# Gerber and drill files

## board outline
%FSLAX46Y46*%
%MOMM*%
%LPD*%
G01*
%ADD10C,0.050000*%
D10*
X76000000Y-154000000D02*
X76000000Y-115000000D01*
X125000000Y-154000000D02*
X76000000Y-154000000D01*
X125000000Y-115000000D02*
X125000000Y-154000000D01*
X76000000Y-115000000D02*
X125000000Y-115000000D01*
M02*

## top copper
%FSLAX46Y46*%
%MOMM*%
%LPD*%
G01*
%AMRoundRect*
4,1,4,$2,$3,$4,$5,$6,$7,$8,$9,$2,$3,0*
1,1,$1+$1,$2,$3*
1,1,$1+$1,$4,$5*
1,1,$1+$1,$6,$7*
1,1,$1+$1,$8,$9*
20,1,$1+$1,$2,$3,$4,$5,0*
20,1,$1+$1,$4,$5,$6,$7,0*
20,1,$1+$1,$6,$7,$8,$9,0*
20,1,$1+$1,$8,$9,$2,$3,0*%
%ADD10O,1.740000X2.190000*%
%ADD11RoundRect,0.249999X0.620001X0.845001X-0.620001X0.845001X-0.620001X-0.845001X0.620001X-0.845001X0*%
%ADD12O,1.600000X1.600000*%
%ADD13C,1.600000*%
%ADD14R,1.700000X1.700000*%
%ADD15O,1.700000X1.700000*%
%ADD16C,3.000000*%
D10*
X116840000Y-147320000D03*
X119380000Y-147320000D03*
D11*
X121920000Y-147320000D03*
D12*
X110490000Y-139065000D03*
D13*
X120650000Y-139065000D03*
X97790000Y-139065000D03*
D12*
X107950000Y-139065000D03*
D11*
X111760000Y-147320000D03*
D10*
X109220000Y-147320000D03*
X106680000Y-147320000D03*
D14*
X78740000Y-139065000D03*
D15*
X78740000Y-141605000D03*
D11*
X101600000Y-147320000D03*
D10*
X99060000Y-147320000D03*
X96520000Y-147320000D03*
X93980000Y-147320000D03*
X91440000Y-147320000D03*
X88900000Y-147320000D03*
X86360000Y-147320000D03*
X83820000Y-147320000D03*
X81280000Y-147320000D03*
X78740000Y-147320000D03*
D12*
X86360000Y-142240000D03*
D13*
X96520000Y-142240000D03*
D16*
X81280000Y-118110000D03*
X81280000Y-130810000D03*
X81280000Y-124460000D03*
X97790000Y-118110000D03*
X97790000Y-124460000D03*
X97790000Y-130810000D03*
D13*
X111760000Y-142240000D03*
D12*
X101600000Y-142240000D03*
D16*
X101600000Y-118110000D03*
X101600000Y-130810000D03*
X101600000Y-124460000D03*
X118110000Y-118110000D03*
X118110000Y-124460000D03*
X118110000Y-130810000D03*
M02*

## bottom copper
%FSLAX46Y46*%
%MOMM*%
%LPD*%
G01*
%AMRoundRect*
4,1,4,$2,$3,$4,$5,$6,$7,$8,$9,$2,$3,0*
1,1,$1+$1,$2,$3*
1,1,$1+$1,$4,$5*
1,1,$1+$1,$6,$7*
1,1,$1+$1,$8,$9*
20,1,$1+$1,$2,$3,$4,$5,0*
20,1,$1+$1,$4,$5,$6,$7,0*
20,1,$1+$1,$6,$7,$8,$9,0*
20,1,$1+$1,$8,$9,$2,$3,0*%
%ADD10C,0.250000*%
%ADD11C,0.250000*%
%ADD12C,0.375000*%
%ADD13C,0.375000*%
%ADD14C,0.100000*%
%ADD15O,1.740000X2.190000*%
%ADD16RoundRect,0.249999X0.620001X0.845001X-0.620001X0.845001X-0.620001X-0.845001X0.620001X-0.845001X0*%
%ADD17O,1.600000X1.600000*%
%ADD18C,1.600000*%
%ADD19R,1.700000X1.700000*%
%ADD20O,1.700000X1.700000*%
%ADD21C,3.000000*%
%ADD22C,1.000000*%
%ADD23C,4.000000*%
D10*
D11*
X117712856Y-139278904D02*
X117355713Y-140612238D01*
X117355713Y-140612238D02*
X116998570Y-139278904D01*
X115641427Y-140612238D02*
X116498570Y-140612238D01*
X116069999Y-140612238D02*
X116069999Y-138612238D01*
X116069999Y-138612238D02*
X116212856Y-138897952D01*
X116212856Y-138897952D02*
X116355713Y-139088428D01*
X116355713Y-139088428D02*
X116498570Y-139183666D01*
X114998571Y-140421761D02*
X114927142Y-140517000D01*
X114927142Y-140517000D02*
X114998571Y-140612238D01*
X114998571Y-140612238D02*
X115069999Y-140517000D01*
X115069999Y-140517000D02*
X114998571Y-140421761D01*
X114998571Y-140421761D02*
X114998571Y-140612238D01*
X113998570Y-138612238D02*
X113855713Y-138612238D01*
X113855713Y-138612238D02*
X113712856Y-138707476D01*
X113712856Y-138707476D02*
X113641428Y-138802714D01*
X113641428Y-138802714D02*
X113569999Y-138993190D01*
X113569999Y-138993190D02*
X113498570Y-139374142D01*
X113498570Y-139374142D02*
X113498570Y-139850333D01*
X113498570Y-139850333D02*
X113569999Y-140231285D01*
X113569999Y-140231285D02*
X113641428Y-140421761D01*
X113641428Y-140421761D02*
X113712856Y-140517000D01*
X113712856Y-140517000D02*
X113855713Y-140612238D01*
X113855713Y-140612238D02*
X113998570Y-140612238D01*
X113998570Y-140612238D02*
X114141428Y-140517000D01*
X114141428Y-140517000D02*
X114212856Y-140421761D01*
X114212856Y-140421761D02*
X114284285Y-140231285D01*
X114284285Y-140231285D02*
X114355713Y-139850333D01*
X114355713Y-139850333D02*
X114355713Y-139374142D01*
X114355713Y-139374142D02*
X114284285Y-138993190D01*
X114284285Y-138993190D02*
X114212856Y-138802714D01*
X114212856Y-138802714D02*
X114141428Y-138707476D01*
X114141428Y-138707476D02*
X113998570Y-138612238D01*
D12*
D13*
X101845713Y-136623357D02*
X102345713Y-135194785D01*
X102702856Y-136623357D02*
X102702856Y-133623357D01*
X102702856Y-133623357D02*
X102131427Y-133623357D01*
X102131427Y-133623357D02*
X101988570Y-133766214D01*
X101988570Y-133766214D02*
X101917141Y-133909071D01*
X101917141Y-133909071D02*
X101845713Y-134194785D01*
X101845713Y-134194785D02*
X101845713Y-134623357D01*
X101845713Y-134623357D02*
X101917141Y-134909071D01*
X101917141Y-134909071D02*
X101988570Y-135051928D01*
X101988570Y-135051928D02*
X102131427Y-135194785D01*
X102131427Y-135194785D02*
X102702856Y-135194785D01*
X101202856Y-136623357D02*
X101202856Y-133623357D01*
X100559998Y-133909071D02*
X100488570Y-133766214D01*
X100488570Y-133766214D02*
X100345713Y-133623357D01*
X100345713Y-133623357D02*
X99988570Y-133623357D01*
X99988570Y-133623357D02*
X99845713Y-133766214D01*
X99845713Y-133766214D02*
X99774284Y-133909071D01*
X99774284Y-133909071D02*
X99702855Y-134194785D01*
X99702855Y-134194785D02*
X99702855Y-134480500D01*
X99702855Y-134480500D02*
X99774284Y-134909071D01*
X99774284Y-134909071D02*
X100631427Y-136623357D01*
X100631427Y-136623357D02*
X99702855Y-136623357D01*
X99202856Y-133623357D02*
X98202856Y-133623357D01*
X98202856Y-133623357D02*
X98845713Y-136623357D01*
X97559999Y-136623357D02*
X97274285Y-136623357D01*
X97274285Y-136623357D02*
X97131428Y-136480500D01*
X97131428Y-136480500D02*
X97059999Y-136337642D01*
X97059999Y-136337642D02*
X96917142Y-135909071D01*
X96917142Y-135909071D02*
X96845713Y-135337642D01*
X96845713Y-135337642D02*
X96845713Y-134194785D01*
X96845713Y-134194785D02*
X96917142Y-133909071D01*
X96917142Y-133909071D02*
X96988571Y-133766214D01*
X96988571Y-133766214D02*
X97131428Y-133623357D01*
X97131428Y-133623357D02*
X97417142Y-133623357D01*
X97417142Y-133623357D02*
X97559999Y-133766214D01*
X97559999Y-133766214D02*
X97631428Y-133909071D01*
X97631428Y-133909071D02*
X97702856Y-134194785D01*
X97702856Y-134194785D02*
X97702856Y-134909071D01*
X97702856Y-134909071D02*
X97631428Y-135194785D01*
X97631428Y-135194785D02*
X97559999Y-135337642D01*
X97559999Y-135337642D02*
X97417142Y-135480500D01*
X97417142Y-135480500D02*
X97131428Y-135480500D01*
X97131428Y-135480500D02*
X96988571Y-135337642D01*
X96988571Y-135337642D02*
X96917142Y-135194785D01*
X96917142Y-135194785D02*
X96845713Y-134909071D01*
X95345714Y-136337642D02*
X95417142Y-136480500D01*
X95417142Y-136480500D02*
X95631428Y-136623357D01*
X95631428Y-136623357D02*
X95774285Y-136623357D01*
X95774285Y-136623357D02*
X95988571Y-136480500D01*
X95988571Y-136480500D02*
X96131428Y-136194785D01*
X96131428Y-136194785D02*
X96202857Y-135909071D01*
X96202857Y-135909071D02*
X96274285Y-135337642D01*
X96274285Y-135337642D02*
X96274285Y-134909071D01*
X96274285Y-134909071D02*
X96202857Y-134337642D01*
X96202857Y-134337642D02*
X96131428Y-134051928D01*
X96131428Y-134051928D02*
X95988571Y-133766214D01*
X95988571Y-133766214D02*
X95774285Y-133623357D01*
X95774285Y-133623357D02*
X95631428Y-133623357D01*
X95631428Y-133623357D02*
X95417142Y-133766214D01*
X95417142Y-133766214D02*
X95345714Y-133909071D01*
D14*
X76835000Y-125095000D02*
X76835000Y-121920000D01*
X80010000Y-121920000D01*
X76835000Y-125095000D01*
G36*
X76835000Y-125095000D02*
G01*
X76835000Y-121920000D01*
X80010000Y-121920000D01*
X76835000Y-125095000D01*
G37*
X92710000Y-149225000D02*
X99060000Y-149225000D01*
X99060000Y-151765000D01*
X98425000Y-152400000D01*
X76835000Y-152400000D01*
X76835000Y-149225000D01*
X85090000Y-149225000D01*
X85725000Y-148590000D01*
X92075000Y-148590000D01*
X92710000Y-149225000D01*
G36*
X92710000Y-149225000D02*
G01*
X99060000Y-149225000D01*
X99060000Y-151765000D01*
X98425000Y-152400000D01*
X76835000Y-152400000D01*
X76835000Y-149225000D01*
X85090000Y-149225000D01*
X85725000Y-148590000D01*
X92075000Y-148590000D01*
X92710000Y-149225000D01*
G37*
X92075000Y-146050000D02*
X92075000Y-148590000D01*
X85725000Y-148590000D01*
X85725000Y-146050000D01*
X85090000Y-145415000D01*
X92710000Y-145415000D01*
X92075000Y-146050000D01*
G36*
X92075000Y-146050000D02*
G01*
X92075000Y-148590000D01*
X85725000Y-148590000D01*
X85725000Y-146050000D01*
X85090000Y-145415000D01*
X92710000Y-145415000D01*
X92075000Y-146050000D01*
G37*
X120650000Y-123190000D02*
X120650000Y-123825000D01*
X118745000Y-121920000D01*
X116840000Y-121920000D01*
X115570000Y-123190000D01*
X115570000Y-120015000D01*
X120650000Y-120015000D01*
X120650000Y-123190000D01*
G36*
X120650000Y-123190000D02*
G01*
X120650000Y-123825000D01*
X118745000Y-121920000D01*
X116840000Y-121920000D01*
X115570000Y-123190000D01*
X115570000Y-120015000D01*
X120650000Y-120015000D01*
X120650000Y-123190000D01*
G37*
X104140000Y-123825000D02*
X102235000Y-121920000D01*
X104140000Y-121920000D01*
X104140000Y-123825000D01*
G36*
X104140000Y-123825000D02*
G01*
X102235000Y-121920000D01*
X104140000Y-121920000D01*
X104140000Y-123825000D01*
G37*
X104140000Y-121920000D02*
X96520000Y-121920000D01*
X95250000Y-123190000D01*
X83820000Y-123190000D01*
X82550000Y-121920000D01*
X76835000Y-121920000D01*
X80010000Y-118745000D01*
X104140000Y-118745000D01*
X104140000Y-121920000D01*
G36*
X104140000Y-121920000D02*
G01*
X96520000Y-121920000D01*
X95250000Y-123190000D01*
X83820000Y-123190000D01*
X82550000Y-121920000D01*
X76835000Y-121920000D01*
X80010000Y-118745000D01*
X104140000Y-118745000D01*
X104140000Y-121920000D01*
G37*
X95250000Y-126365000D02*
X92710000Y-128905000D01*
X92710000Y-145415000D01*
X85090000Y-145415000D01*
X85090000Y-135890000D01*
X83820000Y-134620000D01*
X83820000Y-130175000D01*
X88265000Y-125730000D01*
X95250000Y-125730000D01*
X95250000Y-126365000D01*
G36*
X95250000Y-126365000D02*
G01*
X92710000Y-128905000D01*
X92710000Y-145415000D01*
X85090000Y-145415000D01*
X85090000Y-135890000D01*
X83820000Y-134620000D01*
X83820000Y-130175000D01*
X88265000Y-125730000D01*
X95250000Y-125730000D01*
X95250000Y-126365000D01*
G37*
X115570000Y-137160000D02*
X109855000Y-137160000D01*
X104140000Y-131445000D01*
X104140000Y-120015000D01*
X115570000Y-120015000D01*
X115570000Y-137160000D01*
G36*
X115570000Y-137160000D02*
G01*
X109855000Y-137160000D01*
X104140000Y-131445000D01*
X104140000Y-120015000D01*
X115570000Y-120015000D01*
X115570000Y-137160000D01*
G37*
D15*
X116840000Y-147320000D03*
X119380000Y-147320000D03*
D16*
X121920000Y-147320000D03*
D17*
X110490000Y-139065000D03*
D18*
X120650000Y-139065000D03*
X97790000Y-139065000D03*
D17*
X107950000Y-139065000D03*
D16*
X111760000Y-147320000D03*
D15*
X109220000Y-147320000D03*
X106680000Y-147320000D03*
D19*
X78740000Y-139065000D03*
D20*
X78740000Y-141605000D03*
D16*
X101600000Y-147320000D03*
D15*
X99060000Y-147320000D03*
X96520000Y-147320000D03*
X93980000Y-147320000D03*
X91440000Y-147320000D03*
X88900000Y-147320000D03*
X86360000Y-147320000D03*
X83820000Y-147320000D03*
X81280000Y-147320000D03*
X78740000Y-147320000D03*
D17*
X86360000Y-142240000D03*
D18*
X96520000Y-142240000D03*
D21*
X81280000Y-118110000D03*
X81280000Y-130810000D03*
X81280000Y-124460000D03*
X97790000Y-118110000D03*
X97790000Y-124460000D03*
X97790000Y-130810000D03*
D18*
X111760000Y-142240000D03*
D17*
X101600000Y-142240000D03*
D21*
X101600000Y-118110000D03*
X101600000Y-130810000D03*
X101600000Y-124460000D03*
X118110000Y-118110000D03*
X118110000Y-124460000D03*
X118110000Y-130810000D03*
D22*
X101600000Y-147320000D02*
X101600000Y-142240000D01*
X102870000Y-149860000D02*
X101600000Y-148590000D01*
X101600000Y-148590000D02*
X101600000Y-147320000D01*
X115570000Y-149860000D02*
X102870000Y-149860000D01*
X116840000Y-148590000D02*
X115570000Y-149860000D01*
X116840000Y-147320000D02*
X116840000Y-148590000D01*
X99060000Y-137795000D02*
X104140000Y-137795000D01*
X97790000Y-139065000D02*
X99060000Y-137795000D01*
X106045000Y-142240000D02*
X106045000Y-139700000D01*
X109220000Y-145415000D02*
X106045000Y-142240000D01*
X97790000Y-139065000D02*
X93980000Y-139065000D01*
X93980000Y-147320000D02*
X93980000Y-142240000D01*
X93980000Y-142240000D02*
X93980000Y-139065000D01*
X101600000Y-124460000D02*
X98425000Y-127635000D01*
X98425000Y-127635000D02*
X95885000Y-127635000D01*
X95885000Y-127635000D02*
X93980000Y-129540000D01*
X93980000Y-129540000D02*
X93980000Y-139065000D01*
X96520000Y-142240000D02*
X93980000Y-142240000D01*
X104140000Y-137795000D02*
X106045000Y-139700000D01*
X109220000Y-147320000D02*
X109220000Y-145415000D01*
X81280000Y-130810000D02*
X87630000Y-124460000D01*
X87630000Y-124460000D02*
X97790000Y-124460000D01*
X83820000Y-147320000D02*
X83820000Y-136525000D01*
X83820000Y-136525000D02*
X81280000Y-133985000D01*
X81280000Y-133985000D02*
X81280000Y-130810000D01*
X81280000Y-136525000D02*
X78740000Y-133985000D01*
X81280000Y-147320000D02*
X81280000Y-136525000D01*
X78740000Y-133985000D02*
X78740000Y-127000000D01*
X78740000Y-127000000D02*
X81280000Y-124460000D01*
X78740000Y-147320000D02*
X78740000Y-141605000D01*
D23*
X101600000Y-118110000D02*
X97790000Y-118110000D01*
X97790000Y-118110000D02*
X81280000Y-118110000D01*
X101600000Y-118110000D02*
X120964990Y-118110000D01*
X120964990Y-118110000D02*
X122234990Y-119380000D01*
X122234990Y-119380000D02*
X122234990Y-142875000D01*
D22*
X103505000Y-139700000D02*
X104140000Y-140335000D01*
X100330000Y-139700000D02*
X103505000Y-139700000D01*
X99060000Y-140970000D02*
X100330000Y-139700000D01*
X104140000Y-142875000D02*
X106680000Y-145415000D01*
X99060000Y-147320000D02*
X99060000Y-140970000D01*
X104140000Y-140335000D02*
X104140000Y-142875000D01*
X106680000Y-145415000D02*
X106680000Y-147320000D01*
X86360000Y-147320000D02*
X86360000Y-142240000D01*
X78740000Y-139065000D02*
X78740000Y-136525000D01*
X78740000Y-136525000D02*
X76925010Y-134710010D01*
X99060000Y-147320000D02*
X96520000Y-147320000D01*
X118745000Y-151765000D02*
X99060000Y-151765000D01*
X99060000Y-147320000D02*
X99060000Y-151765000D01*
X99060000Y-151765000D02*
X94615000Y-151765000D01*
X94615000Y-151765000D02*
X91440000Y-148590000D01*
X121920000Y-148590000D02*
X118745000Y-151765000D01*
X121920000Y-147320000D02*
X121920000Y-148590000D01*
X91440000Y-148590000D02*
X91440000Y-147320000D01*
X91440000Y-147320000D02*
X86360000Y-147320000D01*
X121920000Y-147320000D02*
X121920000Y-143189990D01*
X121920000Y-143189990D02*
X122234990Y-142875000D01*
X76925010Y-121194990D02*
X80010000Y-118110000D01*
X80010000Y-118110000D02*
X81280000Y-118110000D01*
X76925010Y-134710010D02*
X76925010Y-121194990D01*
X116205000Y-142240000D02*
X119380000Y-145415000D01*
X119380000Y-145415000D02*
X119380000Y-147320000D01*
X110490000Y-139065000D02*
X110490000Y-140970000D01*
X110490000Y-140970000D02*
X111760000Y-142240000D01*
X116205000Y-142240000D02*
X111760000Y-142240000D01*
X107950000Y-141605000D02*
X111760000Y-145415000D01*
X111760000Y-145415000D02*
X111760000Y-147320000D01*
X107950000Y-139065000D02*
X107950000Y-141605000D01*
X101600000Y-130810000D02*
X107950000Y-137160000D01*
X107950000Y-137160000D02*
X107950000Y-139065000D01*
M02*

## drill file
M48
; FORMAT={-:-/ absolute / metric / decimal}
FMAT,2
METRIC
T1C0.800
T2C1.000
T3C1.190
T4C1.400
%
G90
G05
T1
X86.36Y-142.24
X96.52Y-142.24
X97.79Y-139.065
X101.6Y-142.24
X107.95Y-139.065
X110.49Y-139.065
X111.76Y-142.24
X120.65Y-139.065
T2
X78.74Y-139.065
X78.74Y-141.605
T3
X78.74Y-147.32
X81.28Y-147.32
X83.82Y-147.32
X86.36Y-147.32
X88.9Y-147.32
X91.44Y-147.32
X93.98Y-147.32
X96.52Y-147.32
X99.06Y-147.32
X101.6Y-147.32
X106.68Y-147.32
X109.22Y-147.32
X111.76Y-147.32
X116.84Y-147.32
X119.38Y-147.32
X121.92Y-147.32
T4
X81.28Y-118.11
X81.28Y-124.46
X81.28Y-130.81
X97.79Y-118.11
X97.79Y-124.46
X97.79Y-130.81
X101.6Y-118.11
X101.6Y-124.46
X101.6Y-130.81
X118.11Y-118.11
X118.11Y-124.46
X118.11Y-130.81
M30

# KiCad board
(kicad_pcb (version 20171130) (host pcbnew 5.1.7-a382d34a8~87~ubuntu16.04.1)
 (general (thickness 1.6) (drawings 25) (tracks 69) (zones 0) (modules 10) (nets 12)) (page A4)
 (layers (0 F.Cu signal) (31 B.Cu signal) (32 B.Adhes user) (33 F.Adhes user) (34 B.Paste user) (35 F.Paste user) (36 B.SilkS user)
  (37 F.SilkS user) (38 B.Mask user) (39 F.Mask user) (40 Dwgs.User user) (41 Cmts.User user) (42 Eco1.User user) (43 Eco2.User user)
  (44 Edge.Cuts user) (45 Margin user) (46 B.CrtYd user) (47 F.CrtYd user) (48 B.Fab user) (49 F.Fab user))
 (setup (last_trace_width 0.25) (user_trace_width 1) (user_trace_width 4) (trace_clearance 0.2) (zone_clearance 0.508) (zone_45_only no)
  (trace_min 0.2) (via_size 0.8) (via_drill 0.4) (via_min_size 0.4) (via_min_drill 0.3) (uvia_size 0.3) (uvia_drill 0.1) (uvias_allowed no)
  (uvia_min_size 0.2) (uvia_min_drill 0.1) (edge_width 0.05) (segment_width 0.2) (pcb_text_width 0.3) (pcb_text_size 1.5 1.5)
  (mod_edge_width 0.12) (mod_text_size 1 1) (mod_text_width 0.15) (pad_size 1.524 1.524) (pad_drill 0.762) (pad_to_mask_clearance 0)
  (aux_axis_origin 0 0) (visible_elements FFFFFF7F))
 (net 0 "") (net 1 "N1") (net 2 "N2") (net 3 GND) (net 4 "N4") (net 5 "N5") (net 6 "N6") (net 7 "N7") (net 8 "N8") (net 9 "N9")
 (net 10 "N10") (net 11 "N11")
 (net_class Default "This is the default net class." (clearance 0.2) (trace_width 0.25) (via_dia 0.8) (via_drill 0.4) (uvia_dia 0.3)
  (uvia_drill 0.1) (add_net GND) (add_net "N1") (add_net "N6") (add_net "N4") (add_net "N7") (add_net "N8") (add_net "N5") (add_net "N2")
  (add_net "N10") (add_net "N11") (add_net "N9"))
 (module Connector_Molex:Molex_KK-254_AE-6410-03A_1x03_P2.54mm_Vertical (layer F.Cu) (at 121.92 147.32 180)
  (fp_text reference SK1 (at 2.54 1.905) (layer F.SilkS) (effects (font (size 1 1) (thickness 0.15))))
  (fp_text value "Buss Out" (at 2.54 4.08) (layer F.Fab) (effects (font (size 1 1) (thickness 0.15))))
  (pad 3 thru_hole oval (at 5.08 0 180) (size 1.74 2.19) (drill 1.19) (layers *.Cu *.Mask) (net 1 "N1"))
  (pad 2 thru_hole oval (at 2.54 0 180) (size 1.74 2.19) (drill 1.19) (layers *.Cu *.Mask) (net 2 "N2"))
  (pad 1 thru_hole roundrect (at 0 0 180) (size 1.74 2.19) (drill 1.19) (layers *.Cu *.Mask) (roundrect_rratio 0.1436775862068966)
   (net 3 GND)))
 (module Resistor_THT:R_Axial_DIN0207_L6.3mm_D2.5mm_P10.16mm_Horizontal (layer F.Cu) (at 120.65 139.065 180)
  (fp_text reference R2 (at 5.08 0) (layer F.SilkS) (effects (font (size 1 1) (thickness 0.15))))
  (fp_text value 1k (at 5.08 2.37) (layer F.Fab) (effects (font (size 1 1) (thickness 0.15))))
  (pad 2 thru_hole oval (at 10.16 0 180) (size 1.6 1.6) (drill 0.8) (layers *.Cu *.Mask) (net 2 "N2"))
  (pad 1 thru_hole circle (at 0 0 180) (size 1.6 1.6) (drill 0.8) (layers *.Cu *.Mask) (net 3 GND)))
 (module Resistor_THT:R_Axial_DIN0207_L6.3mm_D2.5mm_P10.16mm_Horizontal (layer F.Cu) (at 97.79 139.065)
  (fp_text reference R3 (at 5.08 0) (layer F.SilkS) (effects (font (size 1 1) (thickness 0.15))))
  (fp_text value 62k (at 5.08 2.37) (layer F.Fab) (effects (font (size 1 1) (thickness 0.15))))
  (pad 1 thru_hole circle (at 0 0) (size 1.6 1.6) (drill 0.8) (layers *.Cu *.Mask) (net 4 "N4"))
  (pad 2 thru_hole oval (at 10.16 0) (size 1.6 1.6) (drill 0.8) (layers *.Cu *.Mask) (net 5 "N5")))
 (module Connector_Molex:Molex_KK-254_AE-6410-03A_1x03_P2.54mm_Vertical (layer F.Cu) (at 111.76 147.32 180)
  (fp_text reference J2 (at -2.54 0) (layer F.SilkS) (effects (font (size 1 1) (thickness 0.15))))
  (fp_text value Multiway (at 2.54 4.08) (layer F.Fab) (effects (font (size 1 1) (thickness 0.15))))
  (pad 1 thru_hole roundrect (at 0 0 180) (size 1.74 2.19) (drill 1.19) (layers *.Cu *.Mask) (roundrect_rratio 0.1436775862068966)
   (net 5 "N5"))
  (pad 2 thru_hole oval (at 2.54 0 180) (size 1.74 2.19) (drill 1.19) (layers *.Cu *.Mask) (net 4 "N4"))
  (pad 3 thru_hole oval (at 5.08 0 180) (size 1.74 2.19) (drill 1.19) (layers *.Cu *.Mask) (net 3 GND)))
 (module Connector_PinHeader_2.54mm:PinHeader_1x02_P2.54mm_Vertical (layer F.Cu) (at 78.74 139.065)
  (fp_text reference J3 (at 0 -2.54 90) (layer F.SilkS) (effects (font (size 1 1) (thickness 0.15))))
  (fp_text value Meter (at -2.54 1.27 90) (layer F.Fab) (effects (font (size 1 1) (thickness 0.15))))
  (pad 1 thru_hole rect (at 0 0) (size 1.7 1.7) (drill 1) (layers *.Cu *.Mask) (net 3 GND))
  (pad 2 thru_hole oval (at 0 2.54) (size 1.7 1.7) (drill 1) (layers *.Cu *.Mask) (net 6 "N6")))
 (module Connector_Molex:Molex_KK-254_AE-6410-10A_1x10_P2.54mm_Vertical (layer F.Cu) (at 101.6 147.32 180)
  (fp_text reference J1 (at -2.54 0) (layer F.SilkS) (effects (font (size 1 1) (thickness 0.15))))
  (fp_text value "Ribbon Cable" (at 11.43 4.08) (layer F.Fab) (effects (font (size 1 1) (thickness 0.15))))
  (pad 1 thru_hole roundrect (at 0 0 180) (size 1.74 2.19) (drill 1.19) (layers *.Cu *.Mask) (roundrect_rratio 0.1436775862068966)
   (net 1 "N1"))
  (pad 2 thru_hole oval (at 2.54 0 180) (size 1.74 2.19) (drill 1.19) (layers *.Cu *.Mask) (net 3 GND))
  (pad 3 thru_hole oval (at 5.08 0 180) (size 1.74 2.19) (drill 1.19) (layers *.Cu *.Mask) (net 3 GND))
  (pad 4 thru_hole oval (at 7.62 0 180) (size 1.74 2.19) (drill 1.19) (layers *.Cu *.Mask) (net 4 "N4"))
  (pad 5 thru_hole oval (at 10.16 0 180) (size 1.74 2.19) (drill 1.19) (layers *.Cu *.Mask) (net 3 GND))
  (pad 6 thru_hole oval (at 12.7 0 180) (size 1.74 2.19) (drill 1.19) (layers *.Cu *.Mask) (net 3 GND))
  (pad 7 thru_hole oval (at 15.24 0 180) (size 1.74 2.19) (drill 1.19) (layers *.Cu *.Mask) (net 3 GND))
  (pad 8 thru_hole oval (at 17.78 0 180) (size 1.74 2.19) (drill 1.19) (layers *.Cu *.Mask) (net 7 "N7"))
  (pad 9 thru_hole oval (at 20.32 0 180) (size 1.74 2.19) (drill 1.19) (layers *.Cu *.Mask) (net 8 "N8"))
  (pad 10 thru_hole oval (at 22.86 0 180) (size 1.74 2.19) (drill 1.19) (layers *.Cu *.Mask) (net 6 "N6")))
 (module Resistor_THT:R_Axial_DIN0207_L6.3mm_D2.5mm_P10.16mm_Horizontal (layer F.Cu) (at 96.52 142.24 180)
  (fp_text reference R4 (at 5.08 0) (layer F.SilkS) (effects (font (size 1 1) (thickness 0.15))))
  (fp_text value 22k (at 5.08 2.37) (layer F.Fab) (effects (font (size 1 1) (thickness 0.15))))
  (pad 2 thru_hole oval (at 10.16 0 180) (size 1.6 1.6) (drill 0.8) (layers *.Cu *.Mask) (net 3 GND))
  (pad 1 thru_hole circle (at 0 0 180) (size 1.6 1.6) (drill 0.8) (layers *.Cu *.Mask) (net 4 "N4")))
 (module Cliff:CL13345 (layer F.Cu) (at 89.535 118.11 90)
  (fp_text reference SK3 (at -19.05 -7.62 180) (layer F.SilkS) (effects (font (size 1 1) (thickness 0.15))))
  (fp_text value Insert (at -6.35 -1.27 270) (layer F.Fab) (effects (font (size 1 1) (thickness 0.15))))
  (pad S thru_hole circle (at 0 -8.255 180) (size 3 3) (drill 1.4) (layers *.Cu *.Mask) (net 3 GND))
  (pad T thru_hole circle (at -12.7 -8.255 180) (size 3 3) (drill 1.4) (layers *.Cu *.Mask) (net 7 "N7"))
  (pad R thru_hole circle (at -6.35 -8.255 180) (size 3 3) (drill 1.4) (layers *.Cu *.Mask) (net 8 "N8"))
  (pad SN thru_hole circle (at 0 8.255 180) (size 3 3) (drill 1.4) (layers *.Cu *.Mask) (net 3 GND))
  (pad RN thru_hole circle (at -6.35 8.255 180) (size 3 3) (drill 1.4) (layers *.Cu *.Mask) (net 7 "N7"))
  (pad TN thru_hole circle (at -12.7 8.255 180) (size 3 3) (drill 1.4) (layers *.Cu *.Mask) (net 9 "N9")))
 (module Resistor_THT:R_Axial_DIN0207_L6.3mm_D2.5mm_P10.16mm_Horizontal (layer F.Cu) (at 111.76 142.24 180)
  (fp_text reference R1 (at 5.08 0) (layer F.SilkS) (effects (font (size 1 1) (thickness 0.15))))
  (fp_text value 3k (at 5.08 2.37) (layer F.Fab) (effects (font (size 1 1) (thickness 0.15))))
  (pad 1 thru_hole circle (at 0 0 180) (size 1.6 1.6) (drill 0.8) (layers *.Cu *.Mask) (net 2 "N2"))
  (pad 2 thru_hole oval (at 10.16 0 180) (size 1.6 1.6) (drill 0.8) (layers *.Cu *.Mask) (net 1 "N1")))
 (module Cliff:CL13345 (layer F.Cu) (at 109.855 118.11 90)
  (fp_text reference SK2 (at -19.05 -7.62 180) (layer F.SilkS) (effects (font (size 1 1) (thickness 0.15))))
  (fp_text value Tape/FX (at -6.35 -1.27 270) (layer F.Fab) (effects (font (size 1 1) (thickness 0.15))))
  (pad S thru_hole circle (at 0 -8.255 180) (size 3 3) (drill 1.4) (layers *.Cu *.Mask) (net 3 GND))
  (pad T thru_hole circle (at -12.7 -8.255 180) (size 3 3) (drill 1.4) (layers *.Cu *.Mask) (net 5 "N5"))
  (pad R thru_hole circle (at -6.35 -8.255 180) (size 3 3) (drill 1.4) (layers *.Cu *.Mask) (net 4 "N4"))
  (pad SN thru_hole circle (at 0 8.255 180) (size 3 3) (drill 1.4) (layers *.Cu *.Mask) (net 3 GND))
  (pad RN thru_hole circle (at -6.35 8.255 180) (size 3 3) (drill 1.4) (layers *.Cu *.Mask) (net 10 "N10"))
  (pad TN thru_hole circle (at -12.7 8.255 180) (size 3 3) (drill 1.4) (layers *.Cu *.Mask) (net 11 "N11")))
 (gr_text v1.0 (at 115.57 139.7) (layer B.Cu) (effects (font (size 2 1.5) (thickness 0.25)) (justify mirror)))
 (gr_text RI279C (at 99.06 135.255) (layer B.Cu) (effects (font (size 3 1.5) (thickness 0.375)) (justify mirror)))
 (gr_poly (pts (xy 76.835 125.095) (xy 76.835 121.92) (xy 80.01 121.92)) (layer B.Cu) (width 0.1))
 (gr_poly
  (pts (xy 92.71 149.225) (xy 99.06 149.225) (xy 99.06 151.765) (xy 98.425 152.4) (xy 76.835 152.4) (xy 76.835 149.225) (xy 85.09 149.225)
   (xy 85.725 148.59) (xy 92.075 148.59))
  (layer B.Cu) (width 0.1))
 (gr_poly
  (pts (xy 92.075 146.05) (xy 92.075 148.59) (xy 85.725 148.59) (xy 85.725 146.05) (xy 85.09 145.415) (xy 92.71 145.415)) (layer B.Cu)
  (width 0.1))
 (gr_poly
  (pts (xy 120.65 123.19) (xy 120.65 123.825) (xy 118.745 121.92) (xy 116.84 121.92) (xy 115.57 123.19) (xy 115.57 120.015)
   (xy 120.65 120.015))
  (layer B.Cu) (width 0.1))
 (gr_poly (pts (xy 104.14 123.825) (xy 102.235 121.92) (xy 104.14 121.92)) (layer B.Cu) (width 0.1))
 (gr_poly
  (pts (xy 104.14 121.92) (xy 96.52 121.92) (xy 95.25 123.19) (xy 83.82 123.19) (xy 82.55 121.92) (xy 76.835 121.92) (xy 80.01 118.745)
   (xy 104.14 118.745))
  (layer B.Cu) (width 0.1))
 (gr_poly
  (pts (xy 95.25 126.365) (xy 92.71 128.905) (xy 92.71 145.415) (xy 85.09 145.415) (xy 85.09 135.89) (xy 83.82 134.62) (xy 83.82 130.175)
   (xy 88.265 125.73) (xy 95.25 125.73))
  (layer B.Cu) (width 0.1))
 (gr_poly (pts (xy 115.57 137.16) (xy 109.855 137.16) (xy 104.14 131.445) (xy 104.14 120.015) (xy 115.57 120.015)) (layer B.Cu) (width 0.1))
 (gr_line (start 76 154) (end 76 115) (layer Edge.Cuts) (width 0.05))
 (gr_line (start 125 154) (end 76 154) (layer Edge.Cuts) (width 0.05))
 (gr_line (start 125 115) (end 125 154) (layer Edge.Cuts) (width 0.05))
 (gr_line (start 76 115) (end 125 115) (layer Edge.Cuts) (width 0.05))
 (segment (start 101.6 147.32) (end 101.6 142.24) (width 1) (layer B.Cu) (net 1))
 (segment (start 102.87 149.86) (end 101.6 148.59) (width 1) (layer B.Cu) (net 1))
 (segment (start 101.6 148.59) (end 101.6 147.32) (width 1) (layer B.Cu) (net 1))
 (segment (start 115.57 149.86) (end 102.87 149.86) (width 1) (layer B.Cu) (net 1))
 (segment (start 116.84 148.59) (end 115.57 149.86) (width 1) (layer B.Cu) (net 1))
 (segment (start 116.84 147.32) (end 116.84 148.59) (width 1) (layer B.Cu) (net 1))
 (segment (start 99.06 137.795) (end 104.14 137.795) (width 1) (layer B.Cu) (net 4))
 (segment (start 97.79 139.065) (end 99.06 137.795) (width 1) (layer B.Cu) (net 4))
 (segment (start 106.045 142.24) (end 106.045 139.7) (width 1) (layer B.Cu) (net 4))
 (segment (start 109.22 145.415) (end 106.045 142.24) (width 1) (layer B.Cu) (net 4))
 (segment (start 97.79 139.065) (end 93.98 139.065) (width 1) (layer B.Cu) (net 4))
 (segment (start 93.98 147.32) (end 93.98 142.24) (width 1) (layer B.Cu) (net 4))
 (segment (start 93.98 142.24) (end 93.98 139.065) (width 1) (layer B.Cu) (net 4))
 (segment (start 101.6 124.46) (end 98.425 127.635) (width 1) (layer B.Cu) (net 4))
 (segment (start 98.425 127.635) (end 95.885 127.635) (width 1) (layer B.Cu) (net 4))
 (segment (start 95.885 127.635) (end 93.98 129.54) (width 1) (layer B.Cu) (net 4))
 (segment (start 93.98 129.54) (end 93.98 139.065) (width 1) (layer B.Cu) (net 4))
 (segment (start 96.52 142.24) (end 93.98 142.24) (width 1) (layer B.Cu) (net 4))
 (segment (start 104.14 137.795) (end 106.045 139.7) (width 1) (layer B.Cu) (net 4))
 (segment (start 109.22 147.32) (end 109.22 145.415) (width 1) (layer B.Cu) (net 4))
 (segment (start 81.28 130.81) (end 87.63 124.46) (width 1) (layer B.Cu) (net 7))
 (segment (start 87.63 124.46) (end 97.79 124.46) (width 1) (layer B.Cu) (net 7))
 (segment (start 83.82 147.32) (end 83.82 136.525) (width 1) (layer B.Cu) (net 7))
 (segment (start 83.82 136.525) (end 81.28 133.985) (width 1) (layer B.Cu) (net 7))
 (segment (start 81.28 133.985) (end 81.28 130.81) (width 1) (layer B.Cu) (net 7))
 (segment (start 81.28 136.525) (end 78.74 133.985) (width 1) (layer B.Cu) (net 8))
 (segment (start 81.28 147.32) (end 81.28 136.525) (width 1) (layer B.Cu) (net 8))
 (segment (start 78.74 133.985) (end 78.74 127) (width 1) (layer B.Cu) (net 8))
 (segment (start 78.74 127) (end 81.28 124.46) (width 1) (layer B.Cu) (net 8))
 (segment (start 78.74 147.32) (end 78.74 141.605) (width 1) (layer B.Cu) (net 6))
 (segment (start 101.6 118.11) (end 97.79 118.11) (width 4) (layer B.Cu) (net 3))
 (segment (start 97.79 118.11) (end 81.28 118.11) (width 4) (layer B.Cu) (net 3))
 (segment (start 101.6 118.11) (end 120.96499 118.11) (width 4) (layer B.Cu) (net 3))
 (segment (start 120.96499 118.11) (end 122.23499 119.38) (width 4) (layer B.Cu) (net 3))
 (segment (start 122.23499 119.38) (end 122.23499 142.875) (width 4) (layer B.Cu) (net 3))
 (segment (start 103.505 139.7) (end 104.14 140.335) (width 1) (layer B.Cu) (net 3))
 (segment (start 100.33 139.7) (end 103.505 139.7) (width 1) (layer B.Cu) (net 3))
 (segment (start 99.06 140.97) (end 100.33 139.7) (width 1) (layer B.Cu) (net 3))
 (segment (start 104.14 142.875) (end 106.68 145.415) (width 1) (layer B.Cu) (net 3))
 (segment (start 99.06 147.32) (end 99.06 140.97) (width 1) (layer B.Cu) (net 3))
 (segment (start 104.14 140.335) (end 104.14 142.875) (width 1) (layer B.Cu) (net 3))
 (segment (start 106.68 145.415) (end 106.68 147.32) (width 1) (layer B.Cu) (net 3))
 (segment (start 86.36 147.32) (end 86.36 142.24) (width 1) (layer B.Cu) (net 3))
 (segment (start 78.74 139.065) (end 78.74 136.525) (width 1) (layer B.Cu) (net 3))
 (segment (start 78.74 136.525) (end 76.92501 134.71001) (width 1) (layer B.Cu) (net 3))
 (segment (start 99.06 147.32) (end 96.52 147.32) (width 1) (layer B.Cu) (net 3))
 (segment (start 118.745 151.765) (end 99.06 151.765) (width 1) (layer B.Cu) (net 3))
 (segment (start 99.06 147.32) (end 99.06 151.765) (width 1) (layer B.Cu) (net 3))
 (segment (start 99.06 151.765) (end 94.615 151.765) (width 1) (layer B.Cu) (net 3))
 (segment (start 94.615 151.765) (end 91.44 148.59) (width 1) (layer B.Cu) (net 3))
 (segment (start 121.92 148.59) (end 118.745 151.765) (width 1) (layer B.Cu) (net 3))
 (segment (start 121.92 147.32) (end 121.92 148.59) (width 1) (layer B.Cu) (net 3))
 (segment (start 91.44 148.59) (end 91.44 147.32) (width 1) (layer B.Cu) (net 3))
 (segment (start 91.44 147.32) (end 86.36 147.32) (width 1) (layer B.Cu) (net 3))
 (segment (start 121.92 147.32) (end 121.92 143.18999) (width 1) (layer B.Cu) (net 3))
 (segment (start 121.92 143.18999) (end 122.23499 142.875) (width 1) (layer B.Cu) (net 3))
 (segment (start 76.92501 121.19499) (end 80.01 118.11) (width 1) (layer B.Cu) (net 3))
 (segment (start 80.01 118.11) (end 81.28 118.11) (width 1) (layer B.Cu) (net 3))
 (segment (start 76.92501 134.71001) (end 76.92501 121.19499) (width 1) (layer B.Cu) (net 3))
 (segment (start 116.205 142.24) (end 119.38 145.415) (width 1) (layer B.Cu) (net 2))
 (segment (start 119.38 145.415) (end 119.38 147.32) (width 1) (layer B.Cu) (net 2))
 (segment (start 110.49 139.065) (end 110.49 140.97) (width 1) (layer B.Cu) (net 2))
 (segment (start 110.49 140.97) (end 111.76 142.24) (width 1) (layer B.Cu) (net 2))
 (segment (start 116.205 142.24) (end 111.76 142.24) (width 1) (layer B.Cu) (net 2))
 (segment (start 107.95 141.605) (end 111.76 145.415) (width 1) (layer B.Cu) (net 5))
 (segment (start 111.76 145.415) (end 111.76 147.32) (width 1) (layer B.Cu) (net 5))
 (segment (start 107.95 139.065) (end 107.95 141.605) (width 1) (layer B.Cu) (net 5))
 (segment (start 101.6 130.81) (end 107.95 137.16) (width 1) (layer B.Cu) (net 5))
 (segment (start 107.95 137.16) (end 107.95 139.065) (width 1) (layer B.Cu) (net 5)))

